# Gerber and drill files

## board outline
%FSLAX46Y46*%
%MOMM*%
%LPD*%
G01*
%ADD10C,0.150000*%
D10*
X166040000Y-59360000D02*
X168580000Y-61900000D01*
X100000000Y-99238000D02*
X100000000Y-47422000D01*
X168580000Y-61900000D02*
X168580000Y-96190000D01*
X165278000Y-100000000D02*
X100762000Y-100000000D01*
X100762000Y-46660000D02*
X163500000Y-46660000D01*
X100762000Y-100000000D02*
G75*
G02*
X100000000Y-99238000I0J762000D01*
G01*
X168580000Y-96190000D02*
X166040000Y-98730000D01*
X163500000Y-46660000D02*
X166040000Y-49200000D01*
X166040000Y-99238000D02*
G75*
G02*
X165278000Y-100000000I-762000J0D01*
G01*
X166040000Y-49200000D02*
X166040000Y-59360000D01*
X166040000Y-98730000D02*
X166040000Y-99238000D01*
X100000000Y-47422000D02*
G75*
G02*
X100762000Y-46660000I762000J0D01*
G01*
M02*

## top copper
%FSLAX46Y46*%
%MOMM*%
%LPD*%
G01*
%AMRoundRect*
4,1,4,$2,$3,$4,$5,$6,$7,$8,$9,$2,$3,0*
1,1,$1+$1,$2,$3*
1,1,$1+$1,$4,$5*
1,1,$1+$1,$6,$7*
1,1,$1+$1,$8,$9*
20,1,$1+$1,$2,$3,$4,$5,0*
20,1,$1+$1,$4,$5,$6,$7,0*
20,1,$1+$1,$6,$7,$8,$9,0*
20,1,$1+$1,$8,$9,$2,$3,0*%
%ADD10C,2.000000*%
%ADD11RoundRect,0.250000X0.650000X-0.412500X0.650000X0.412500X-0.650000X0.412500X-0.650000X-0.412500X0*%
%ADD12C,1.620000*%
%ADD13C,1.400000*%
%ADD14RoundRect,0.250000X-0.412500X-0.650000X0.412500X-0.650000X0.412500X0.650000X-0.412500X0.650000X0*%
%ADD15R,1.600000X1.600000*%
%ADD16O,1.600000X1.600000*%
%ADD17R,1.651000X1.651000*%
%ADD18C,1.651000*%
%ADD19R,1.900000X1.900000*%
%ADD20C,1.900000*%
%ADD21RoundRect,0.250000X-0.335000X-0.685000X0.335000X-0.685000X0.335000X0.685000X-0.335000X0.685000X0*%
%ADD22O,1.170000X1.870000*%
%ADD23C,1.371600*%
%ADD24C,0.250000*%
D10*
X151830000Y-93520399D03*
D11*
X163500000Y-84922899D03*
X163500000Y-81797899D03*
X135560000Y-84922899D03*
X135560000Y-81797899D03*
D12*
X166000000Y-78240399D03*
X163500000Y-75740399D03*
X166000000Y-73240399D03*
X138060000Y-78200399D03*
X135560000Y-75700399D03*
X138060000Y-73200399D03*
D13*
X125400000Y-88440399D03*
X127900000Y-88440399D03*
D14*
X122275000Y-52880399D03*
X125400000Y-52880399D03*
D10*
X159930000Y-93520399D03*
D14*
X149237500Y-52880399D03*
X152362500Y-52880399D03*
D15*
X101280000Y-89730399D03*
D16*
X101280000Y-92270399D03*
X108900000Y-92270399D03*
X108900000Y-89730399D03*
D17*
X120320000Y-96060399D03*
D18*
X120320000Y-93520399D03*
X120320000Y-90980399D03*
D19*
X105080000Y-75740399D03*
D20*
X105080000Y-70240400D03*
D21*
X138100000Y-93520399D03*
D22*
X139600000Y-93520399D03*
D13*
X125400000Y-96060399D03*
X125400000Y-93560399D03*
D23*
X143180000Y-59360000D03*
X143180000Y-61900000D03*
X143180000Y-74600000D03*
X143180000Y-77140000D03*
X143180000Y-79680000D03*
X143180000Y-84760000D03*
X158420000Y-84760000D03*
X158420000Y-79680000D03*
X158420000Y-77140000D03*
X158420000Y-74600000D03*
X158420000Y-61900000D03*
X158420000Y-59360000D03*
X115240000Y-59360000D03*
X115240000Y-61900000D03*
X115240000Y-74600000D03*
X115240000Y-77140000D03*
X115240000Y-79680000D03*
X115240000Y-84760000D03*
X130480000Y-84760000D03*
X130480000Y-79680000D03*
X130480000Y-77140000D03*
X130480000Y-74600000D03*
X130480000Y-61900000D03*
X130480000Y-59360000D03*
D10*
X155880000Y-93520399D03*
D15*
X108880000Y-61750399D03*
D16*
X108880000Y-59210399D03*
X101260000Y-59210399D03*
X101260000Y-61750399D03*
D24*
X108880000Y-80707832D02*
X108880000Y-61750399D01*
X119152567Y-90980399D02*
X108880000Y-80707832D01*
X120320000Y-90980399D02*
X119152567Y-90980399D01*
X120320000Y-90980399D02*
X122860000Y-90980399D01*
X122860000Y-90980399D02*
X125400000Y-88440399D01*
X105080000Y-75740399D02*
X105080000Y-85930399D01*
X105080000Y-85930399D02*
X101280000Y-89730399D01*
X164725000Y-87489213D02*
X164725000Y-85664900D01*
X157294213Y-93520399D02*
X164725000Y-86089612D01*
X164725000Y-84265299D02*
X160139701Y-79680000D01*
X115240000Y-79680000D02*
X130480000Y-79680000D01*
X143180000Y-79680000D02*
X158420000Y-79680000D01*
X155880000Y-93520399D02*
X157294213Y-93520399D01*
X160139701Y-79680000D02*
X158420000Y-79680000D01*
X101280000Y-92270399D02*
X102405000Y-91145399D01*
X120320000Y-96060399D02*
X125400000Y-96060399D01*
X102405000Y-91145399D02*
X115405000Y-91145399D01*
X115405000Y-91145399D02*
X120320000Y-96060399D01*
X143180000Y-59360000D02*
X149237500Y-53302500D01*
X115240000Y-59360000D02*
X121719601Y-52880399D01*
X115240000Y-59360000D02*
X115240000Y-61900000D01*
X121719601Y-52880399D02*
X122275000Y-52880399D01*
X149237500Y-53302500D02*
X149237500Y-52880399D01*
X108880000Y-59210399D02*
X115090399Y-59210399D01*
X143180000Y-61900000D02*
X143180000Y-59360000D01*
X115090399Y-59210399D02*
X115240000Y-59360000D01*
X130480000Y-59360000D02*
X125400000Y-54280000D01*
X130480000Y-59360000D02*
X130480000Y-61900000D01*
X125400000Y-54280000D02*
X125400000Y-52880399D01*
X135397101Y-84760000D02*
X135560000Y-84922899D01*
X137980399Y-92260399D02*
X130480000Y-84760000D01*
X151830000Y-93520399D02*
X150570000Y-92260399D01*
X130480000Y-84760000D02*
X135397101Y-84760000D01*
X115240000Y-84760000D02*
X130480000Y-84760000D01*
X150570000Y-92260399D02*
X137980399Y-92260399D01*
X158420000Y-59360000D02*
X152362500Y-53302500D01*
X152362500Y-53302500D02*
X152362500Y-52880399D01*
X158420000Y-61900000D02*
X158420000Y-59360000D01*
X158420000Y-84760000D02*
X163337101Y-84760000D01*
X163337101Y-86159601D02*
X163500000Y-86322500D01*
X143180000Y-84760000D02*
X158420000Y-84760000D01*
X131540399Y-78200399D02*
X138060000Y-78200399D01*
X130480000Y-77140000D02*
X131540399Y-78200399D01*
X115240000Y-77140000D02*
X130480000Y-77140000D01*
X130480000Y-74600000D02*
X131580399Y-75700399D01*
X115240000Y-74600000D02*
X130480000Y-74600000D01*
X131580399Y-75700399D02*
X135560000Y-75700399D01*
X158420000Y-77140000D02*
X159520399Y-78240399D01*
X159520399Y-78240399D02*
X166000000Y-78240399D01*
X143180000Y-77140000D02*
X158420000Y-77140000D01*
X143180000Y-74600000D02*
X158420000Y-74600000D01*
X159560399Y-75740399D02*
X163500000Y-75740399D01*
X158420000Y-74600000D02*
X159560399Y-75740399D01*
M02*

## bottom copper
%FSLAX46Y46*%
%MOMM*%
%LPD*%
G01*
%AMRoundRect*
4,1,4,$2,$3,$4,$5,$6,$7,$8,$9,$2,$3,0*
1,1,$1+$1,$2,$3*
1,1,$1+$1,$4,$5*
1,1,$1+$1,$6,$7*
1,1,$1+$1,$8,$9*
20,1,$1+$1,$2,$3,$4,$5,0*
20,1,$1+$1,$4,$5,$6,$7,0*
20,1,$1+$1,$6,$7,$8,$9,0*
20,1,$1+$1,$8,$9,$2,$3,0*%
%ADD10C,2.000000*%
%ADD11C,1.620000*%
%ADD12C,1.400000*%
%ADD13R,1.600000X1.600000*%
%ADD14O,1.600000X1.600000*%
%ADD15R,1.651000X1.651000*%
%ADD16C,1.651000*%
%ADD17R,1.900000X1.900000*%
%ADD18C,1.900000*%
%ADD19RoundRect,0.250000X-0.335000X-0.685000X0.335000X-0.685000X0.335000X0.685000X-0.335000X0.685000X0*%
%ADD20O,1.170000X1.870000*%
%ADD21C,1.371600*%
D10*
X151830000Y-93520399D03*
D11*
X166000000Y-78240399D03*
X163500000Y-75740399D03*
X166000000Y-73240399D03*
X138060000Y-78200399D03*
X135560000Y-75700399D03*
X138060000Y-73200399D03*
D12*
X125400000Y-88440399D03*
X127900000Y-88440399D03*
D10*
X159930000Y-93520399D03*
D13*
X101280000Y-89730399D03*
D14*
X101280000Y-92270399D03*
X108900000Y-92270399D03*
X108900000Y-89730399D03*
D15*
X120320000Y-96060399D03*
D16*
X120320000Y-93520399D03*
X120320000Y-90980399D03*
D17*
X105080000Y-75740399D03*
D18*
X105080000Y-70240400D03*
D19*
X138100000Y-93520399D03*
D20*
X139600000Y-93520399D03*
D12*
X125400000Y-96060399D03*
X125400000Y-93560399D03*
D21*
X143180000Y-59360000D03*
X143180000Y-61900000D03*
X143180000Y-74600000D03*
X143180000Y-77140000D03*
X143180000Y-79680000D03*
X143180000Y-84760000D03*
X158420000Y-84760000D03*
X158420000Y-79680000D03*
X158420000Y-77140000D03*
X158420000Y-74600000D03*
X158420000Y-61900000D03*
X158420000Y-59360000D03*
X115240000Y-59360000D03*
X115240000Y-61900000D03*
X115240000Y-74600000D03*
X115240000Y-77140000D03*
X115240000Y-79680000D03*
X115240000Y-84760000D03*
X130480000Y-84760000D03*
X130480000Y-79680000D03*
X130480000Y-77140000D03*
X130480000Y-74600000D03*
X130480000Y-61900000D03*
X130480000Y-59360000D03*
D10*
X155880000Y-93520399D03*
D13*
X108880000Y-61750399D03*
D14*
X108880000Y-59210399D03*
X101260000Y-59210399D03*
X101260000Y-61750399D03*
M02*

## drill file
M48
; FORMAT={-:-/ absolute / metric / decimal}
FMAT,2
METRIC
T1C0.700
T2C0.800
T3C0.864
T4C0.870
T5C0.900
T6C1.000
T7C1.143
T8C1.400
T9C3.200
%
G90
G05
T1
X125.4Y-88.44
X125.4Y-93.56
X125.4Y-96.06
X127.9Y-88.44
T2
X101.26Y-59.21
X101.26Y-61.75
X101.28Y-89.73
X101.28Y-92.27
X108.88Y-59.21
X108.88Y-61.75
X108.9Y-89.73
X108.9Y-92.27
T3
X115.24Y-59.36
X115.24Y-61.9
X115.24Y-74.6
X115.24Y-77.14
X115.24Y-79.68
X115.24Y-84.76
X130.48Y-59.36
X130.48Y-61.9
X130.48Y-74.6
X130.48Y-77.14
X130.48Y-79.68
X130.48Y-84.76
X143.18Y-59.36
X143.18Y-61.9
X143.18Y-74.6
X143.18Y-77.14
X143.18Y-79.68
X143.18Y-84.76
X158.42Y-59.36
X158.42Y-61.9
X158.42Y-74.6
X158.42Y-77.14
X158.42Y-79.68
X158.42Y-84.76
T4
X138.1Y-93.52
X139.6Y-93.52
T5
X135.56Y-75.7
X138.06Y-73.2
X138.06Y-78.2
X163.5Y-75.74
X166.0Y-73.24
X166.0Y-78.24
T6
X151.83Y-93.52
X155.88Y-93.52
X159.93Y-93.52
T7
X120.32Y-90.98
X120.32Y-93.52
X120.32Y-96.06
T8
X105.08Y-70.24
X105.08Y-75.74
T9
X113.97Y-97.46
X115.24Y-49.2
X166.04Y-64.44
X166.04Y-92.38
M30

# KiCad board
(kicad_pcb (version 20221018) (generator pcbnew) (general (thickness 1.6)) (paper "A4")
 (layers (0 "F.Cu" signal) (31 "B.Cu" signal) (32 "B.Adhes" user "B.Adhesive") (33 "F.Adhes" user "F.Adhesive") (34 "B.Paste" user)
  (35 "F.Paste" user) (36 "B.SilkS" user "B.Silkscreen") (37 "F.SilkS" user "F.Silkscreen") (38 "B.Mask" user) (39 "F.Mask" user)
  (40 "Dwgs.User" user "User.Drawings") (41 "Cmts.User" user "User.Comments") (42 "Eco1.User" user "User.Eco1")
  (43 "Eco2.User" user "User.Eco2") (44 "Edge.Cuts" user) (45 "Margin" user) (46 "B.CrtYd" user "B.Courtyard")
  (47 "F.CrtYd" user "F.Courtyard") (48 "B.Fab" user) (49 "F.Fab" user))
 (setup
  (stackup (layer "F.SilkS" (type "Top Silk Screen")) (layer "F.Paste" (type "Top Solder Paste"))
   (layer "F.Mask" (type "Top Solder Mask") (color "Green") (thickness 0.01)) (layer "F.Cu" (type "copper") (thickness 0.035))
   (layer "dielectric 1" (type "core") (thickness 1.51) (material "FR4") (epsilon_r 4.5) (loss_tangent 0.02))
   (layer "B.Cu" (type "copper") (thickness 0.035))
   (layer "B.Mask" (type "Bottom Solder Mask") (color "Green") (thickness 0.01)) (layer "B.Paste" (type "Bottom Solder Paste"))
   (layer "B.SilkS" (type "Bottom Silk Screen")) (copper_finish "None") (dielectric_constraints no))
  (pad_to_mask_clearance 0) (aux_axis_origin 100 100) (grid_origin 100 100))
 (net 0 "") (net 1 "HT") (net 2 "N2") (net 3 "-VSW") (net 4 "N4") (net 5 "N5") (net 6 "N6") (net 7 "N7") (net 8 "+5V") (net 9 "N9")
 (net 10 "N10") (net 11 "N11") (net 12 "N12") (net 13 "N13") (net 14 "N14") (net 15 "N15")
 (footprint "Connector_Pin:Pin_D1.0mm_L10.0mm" (layer "F.Cu") (at 151.83 93.520399 90)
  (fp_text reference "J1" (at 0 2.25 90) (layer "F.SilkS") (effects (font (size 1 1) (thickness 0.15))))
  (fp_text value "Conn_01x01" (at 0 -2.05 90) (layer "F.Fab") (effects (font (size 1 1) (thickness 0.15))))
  (pad "1" thru_hole circle (at 0 0 90) (size 2 2) (drill 1) (layers "*.Cu" "*.Mask") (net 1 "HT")))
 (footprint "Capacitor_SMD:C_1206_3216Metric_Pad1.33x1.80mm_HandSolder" (layer "F.Cu") (at 163.5 83.360399 90)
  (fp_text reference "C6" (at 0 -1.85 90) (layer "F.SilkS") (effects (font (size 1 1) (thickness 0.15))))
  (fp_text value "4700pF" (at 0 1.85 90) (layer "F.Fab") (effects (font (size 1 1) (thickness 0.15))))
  (pad "1" smd roundrect (at -1.5625 0 90) (size 1.325 1.8) (layers "F.Cu" "F.Paste" "F.Mask") (roundrect_rratio 0.188679) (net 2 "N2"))
  (pad "2" smd roundrect (at 1.5625 0 90) (size 1.325 1.8) (layers "F.Cu" "F.Paste" "F.Mask") (roundrect_rratio 0.188679) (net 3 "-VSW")))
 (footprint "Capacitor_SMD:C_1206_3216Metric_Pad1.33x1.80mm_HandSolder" (layer "F.Cu") (at 135.56 83.360399 90)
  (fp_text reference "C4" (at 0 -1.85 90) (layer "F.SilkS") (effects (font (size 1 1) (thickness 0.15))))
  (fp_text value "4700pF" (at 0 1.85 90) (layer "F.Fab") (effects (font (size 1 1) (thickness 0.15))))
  (pad "1" smd roundrect (at -1.5625 0 90) (size 1.325 1.8) (layers "F.Cu" "F.Paste" "F.Mask") (roundrect_rratio 0.188679) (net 1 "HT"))
  (pad "2" smd roundrect (at 1.5625 0 90) (size 1.325 1.8) (layers "F.Cu" "F.Paste" "F.Mask") (roundrect_rratio 0.188679) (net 3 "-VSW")))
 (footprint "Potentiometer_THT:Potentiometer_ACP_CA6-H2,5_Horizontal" (layer "F.Cu") (at 166 78.240399 180)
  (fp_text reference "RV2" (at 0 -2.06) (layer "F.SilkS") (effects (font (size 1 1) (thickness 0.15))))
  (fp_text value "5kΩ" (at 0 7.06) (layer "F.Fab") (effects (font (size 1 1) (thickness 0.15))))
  (pad "1" thru_hole circle (at 0 0 180) (size 1.62 1.62) (drill 0.9) (layers "*.Cu" "*.Mask") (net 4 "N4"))
  (pad "2" thru_hole circle (at 2.5 2.5 180) (size 1.62 1.62) (drill 0.9) (layers "*.Cu" "*.Mask") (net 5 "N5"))
  (pad "3" thru_hole circle (at 0 5 180) (size 1.62 1.62) (drill 0.9) (layers "*.Cu" "*.Mask") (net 3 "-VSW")))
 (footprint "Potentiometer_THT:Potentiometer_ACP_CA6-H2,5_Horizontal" (layer "F.Cu") (at 138.06 78.200399 180)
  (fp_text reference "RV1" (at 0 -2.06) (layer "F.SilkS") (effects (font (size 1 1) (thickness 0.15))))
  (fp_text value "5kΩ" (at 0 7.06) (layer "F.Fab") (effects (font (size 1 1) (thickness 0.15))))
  (pad "1" thru_hole circle (at 0 0 180) (size 1.62 1.62) (drill 0.9) (layers "*.Cu" "*.Mask") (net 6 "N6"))
  (pad "2" thru_hole circle (at 2.5 2.5 180) (size 1.62 1.62) (drill 0.9) (layers "*.Cu" "*.Mask") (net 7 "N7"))
  (pad "3" thru_hole circle (at 0 5 180) (size 1.62 1.62) (drill 0.9) (layers "*.Cu" "*.Mask") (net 3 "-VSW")))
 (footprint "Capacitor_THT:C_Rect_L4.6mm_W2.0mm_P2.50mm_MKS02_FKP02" (layer "F.Cu") (at 125.4 88.440399)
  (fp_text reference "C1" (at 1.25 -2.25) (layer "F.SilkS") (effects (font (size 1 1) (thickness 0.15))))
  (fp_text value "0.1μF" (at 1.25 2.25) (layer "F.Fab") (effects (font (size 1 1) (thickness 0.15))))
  (pad "1" thru_hole circle (at 0 0) (size 1.4 1.4) (drill 0.7) (layers "*.Cu" "*.Mask") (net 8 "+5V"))
  (pad "2" thru_hole circle (at 2.5 0) (size 1.4 1.4) (drill 0.7) (layers "*.Cu" "*.Mask") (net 3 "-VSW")))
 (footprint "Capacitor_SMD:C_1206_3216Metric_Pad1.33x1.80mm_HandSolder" (layer "F.Cu") (at 123.8375 52.880399)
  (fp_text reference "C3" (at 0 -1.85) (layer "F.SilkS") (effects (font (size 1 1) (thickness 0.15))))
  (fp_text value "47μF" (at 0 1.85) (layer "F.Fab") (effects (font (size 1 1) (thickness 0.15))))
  (pad "1" smd roundrect (at -1.5625 0) (size 1.325 1.8) (layers "F.Cu" "F.Paste" "F.Mask") (roundrect_rratio 0.188679) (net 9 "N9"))
  (pad "2" smd roundrect (at 1.5625 0) (size 1.325 1.8) (layers "F.Cu" "F.Paste" "F.Mask") (roundrect_rratio 0.188679) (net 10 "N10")))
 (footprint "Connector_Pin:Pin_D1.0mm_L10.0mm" (layer "F.Cu") (at 159.93 93.520399 90)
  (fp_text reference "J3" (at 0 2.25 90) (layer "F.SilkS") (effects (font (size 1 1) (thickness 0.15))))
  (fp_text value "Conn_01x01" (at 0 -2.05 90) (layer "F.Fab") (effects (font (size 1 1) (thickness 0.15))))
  (pad "1" thru_hole circle (at 0 0 90) (size 2 2) (drill 1) (layers "*.Cu" "*.Mask") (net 3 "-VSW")))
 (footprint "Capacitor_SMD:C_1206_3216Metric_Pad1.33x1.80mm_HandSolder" (layer "F.Cu") (at 150.8 52.880399)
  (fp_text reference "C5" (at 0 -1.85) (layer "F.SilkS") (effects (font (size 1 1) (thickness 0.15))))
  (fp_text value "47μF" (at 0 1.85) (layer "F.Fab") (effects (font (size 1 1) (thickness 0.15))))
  (pad "1" smd roundrect (at -1.5625 0) (size 1.325 1.8) (layers "F.Cu" "F.Paste" "F.Mask") (roundrect_rratio 0.188679) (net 9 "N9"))
  (pad "2" smd roundrect (at 1.5625 0) (size 1.325 1.8) (layers "F.Cu" "F.Paste" "F.Mask") (roundrect_rratio 0.188679) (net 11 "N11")))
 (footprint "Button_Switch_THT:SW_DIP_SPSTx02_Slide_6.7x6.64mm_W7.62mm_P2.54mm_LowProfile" (layer "F.Cu") (at 101.28 89.730399)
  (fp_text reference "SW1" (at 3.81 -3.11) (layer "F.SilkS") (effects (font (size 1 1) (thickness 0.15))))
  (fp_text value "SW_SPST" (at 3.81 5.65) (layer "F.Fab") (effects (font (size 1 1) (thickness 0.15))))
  (pad "1" thru_hole rect (at 0 0) (size 1.6 1.6) (drill 0.8) (layers "*.Cu" "*.Mask") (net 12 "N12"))
  (pad "2" thru_hole oval (at 0 2.54) (size 1.6 1.6) (drill 0.8) (layers "*.Cu" "*.Mask") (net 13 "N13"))
  (pad "3" thru_hole oval (at 7.62 2.54) (size 1.6 1.6) (drill 0.8) (layers "*.Cu" "*.Mask"))
  (pad "4" thru_hole oval (at 7.62 0) (size 1.6 1.6) (drill 0.8) (layers "*.Cu" "*.Mask")))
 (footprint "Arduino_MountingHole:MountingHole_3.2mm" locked (layer "F.Cu") (at 115.24 49.2)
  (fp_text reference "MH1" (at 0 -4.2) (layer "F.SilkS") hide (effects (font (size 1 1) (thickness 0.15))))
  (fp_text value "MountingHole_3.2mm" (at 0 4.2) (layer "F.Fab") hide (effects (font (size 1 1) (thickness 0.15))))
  (pad "" np_thru_hole circle locked (at 0 0) (size 3.2 3.2) (drill 3.2) (layers "*.Cu" "*.Mask")))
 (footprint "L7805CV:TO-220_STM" (layer "F.Cu") (at 120.32 96.060399 90)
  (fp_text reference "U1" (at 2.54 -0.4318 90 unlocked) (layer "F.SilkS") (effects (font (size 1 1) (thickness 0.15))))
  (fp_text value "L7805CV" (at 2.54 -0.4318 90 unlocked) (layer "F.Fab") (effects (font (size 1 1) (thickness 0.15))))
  (pad "1" thru_hole rect (at 0 0 90) (size 1.651 1.651) (drill 1.143) (layers "*.Cu" "*.Mask") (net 13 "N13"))
  (pad "2" thru_hole circle (at 2.54 0 90) (size 1.651 1.651) (drill 1.143) (layers "*.Cu" "*.Mask") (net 3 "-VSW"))
  (pad "3" thru_hole circle (at 5.08 0 90) (size 1.651 1.651) (drill 1.143) (layers "*.Cu" "*.Mask") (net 8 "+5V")))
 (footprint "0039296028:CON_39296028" (layer "F.Cu") (at 105.08 75.740399 180)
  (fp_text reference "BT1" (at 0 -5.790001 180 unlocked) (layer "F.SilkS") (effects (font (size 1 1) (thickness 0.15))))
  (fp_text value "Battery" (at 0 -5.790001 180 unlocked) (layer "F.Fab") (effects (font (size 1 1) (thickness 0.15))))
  (pad "1" thru_hole rect (at 0 0 180) (size 1.9 1.9) (drill 1.4) (layers "*.Cu" "*.Mask") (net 12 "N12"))
  (pad "2" thru_hole circle (at 0 5.499999 180) (size 1.9 1.9) (drill 1.4) (layers "*.Cu" "*.Mask") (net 3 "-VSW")))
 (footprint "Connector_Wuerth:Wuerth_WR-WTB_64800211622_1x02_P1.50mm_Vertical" (layer "F.Cu") (at 138.1 93.520399)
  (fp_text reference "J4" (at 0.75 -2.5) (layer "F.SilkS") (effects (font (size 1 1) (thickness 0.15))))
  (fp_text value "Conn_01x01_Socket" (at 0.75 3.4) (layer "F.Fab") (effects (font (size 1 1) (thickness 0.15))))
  (pad "1" thru_hole roundrect (at 0 0) (size 1.17 1.87) (drill 0.87) (layers "*.Cu" "*.Mask") (roundrect_rratio 0.213675) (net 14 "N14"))
  (pad "2" thru_hole oval (at 1.5 0) (size 1.17 1.87) (drill 0.87) (layers "*.Cu" "*.Mask") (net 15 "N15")))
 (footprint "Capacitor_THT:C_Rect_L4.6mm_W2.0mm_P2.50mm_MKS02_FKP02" (layer "F.Cu") (at 125.4 96.060399 90)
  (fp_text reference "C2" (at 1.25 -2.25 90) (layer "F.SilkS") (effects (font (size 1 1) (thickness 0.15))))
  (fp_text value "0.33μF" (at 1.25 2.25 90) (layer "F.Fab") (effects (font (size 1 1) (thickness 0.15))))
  (pad "1" thru_hole circle (at 0 0 90) (size 1.4 1.4) (drill 0.7) (layers "*.Cu" "*.Mask") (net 13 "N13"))
  (pad "2" thru_hole circle (at 2.5 0 90) (size 1.4 1.4) (drill 0.7) (layers "*.Cu" "*.Mask") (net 3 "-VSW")))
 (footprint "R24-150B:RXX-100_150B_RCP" (layer "F.Cu") (at 143.18 59.36)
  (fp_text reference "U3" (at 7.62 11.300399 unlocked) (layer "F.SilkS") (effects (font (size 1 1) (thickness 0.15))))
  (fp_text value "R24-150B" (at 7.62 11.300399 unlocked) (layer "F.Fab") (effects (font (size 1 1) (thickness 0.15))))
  (pad "2" thru_hole circle (at 0 0) (size 1.3716 1.3716) (drill 0.8636) (layers "*.Cu" "*.Mask") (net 9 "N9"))
  (pad "3" thru_hole circle (at 0 2.54) (size 1.3716 1.3716) (drill 0.8636) (layers "*.Cu" "*.Mask") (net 9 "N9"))
  (pad "8" thru_hole circle (at 0 15.24) (size 1.3716 1.3716) (drill 0.8636) (layers "*.Cu" "*.Mask") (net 5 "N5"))
  (pad "9" thru_hole circle (at 0 17.78) (size 1.3716 1.3716) (drill 0.8636) (layers "*.Cu" "*.Mask") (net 4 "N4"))
  (pad "10" thru_hole circle (at 0 20.32) (size 1.3716 1.3716) (drill 0.8636) (layers "*.Cu" "*.Mask") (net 3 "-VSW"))
  (pad "12" thru_hole circle (at 0 25.4) (size 1.3716 1.3716) (drill 0.8636) (layers "*.Cu" "*.Mask") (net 2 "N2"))
  (pad "13" thru_hole circle (at 15.24 25.4) (size 1.3716 1.3716) (drill 0.8636) (layers "*.Cu" "*.Mask") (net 2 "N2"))
  (pad "15" thru_hole circle (at 15.24 20.32) (size 1.3716 1.3716) (drill 0.8636) (layers "*.Cu" "*.Mask") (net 3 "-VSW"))
  (pad "16" thru_hole circle (at 15.24 17.78) (size 1.3716 1.3716) (drill 0.8636) (layers "*.Cu" "*.Mask") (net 4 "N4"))
  (pad "17" thru_hole circle (at 15.24 15.24) (size 1.3716 1.3716) (drill 0.8636) (layers "*.Cu" "*.Mask") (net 5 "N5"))
  (pad "22" thru_hole circle (at 15.24 2.54) (size 1.3716 1.3716) (drill 0.8636) (layers "*.Cu" "*.Mask") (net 11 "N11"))
  (pad "23" thru_hole circle (at 15.24 0) (size 1.3716 1.3716) (drill 0.8636) (layers "*.Cu" "*.Mask") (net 11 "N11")))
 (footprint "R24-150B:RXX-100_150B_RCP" (layer "F.Cu") (at 115.24 59.36)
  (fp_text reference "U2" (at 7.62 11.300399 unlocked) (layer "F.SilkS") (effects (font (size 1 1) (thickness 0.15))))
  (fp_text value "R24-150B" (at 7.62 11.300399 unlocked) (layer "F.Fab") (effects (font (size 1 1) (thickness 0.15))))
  (pad "2" thru_hole circle (at 0 0) (size 1.3716 1.3716) (drill 0.8636) (layers "*.Cu" "*.Mask") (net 9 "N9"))
  (pad "3" thru_hole circle (at 0 2.54) (size 1.3716 1.3716) (drill 0.8636) (layers "*.Cu" "*.Mask") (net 9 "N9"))
  (pad "8" thru_hole circle (at 0 15.24) (size 1.3716 1.3716) (drill 0.8636) (layers "*.Cu" "*.Mask") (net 7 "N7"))
  (pad "9" thru_hole circle (at 0 17.78) (size 1.3716 1.3716) (drill 0.8636) (layers "*.Cu" "*.Mask") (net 6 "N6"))
  (pad "10" thru_hole circle (at 0 20.32) (size 1.3716 1.3716) (drill 0.8636) (layers "*.Cu" "*.Mask") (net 3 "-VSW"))
  (pad "12" thru_hole circle (at 0 25.4) (size 1.3716 1.3716) (drill 0.8636) (layers "*.Cu" "*.Mask") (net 1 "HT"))
  (pad "13" thru_hole circle (at 15.24 25.4) (size 1.3716 1.3716) (drill 0.8636) (layers "*.Cu" "*.Mask") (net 1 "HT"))
  (pad "15" thru_hole circle (at 15.24 20.32) (size 1.3716 1.3716) (drill 0.8636) (layers "*.Cu" "*.Mask") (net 3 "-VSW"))
  (pad "16" thru_hole circle (at 15.24 17.78) (size 1.3716 1.3716) (drill 0.8636) (layers "*.Cu" "*.Mask") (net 6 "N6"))
  (pad "17" thru_hole circle (at 15.24 15.24) (size 1.3716 1.3716) (drill 0.8636) (layers "*.Cu" "*.Mask") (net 7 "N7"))
  (pad "22" thru_hole circle (at 15.24 2.54) (size 1.3716 1.3716) (drill 0.8636) (layers "*.Cu" "*.Mask") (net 10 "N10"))
  (pad "23" thru_hole circle (at 15.24 0) (size 1.3716 1.3716) (drill 0.8636) (layers "*.Cu" "*.Mask") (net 10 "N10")))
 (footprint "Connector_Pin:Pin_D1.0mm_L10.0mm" (layer "F.Cu") (at 155.88 93.520399 90)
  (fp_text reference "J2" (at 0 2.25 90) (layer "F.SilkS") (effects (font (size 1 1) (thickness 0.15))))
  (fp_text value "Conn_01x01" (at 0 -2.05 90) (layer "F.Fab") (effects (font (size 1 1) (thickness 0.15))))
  (pad "1" thru_hole circle (at 0 0 90) (size 2 2) (drill 1) (layers "*.Cu" "*.Mask") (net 3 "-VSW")))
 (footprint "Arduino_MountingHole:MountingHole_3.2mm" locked (layer "F.Cu") (at 113.97 97.46)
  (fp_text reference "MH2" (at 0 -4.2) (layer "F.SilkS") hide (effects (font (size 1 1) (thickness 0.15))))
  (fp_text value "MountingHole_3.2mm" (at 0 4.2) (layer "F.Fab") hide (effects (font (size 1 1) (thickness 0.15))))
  (pad "" np_thru_hole circle locked (at 0 0) (size 3.2 3.2) (drill 3.2) (layers "*.Cu" "*.Mask")))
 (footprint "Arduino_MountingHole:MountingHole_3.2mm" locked (layer "F.Cu") (at 166.04 64.44)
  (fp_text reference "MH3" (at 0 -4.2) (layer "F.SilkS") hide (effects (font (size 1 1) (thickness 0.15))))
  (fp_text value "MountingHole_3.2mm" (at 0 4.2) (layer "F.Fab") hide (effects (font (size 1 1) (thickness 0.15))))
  (pad "" np_thru_hole circle locked (at 0 0) (size 3.2 3.2) (drill 3.2) (layers "*.Cu" "*.Mask")))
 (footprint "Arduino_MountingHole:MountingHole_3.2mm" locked (layer "F.Cu") (at 166.04 92.38)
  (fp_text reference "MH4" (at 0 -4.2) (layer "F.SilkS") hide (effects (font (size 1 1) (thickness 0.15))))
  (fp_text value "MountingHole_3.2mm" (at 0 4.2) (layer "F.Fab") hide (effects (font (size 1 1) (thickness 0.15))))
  (pad "" np_thru_hole circle locked (at 0 0) (size 3.2 3.2) (drill 3.2) (layers "*.Cu" "*.Mask")))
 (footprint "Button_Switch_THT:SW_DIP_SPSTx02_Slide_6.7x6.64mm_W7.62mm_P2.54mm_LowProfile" (layer "F.Cu") (at 108.88 61.750399 180)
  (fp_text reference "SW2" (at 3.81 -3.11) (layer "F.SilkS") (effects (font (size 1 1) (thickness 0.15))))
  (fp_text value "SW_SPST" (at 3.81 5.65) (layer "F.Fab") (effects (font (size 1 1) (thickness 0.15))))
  (pad "1" thru_hole rect (at 0 0 180) (size 1.6 1.6) (drill 0.8) (layers "*.Cu" "*.Mask") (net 8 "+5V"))
  (pad "2" thru_hole oval (at 0 2.54 180) (size 1.6 1.6) (drill 0.8) (layers "*.Cu" "*.Mask") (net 9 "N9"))
  (pad "3" thru_hole oval (at 7.62 2.54 180) (size 1.6 1.6) (drill 0.8) (layers "*.Cu" "*.Mask"))
  (pad "4" thru_hole oval (at 7.62 0 180) (size 1.6 1.6) (drill 0.8) (layers "*.Cu" "*.Mask")))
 (gr_line (start 166.04 59.36) (end 168.58 61.9) (stroke (width 0.15) (type solid)) (layer "Edge.Cuts"))
 (gr_line (start 100 99.238) (end 100 47.422) (stroke (width 0.15) (type solid)) (layer "Edge.Cuts"))
 (gr_line (start 168.58 61.9) (end 168.58 96.19) (stroke (width 0.15) (type solid)) (layer "Edge.Cuts"))
 (gr_line (start 165.278 100) (end 100.762 100) (stroke (width 0.15) (type solid)) (layer "Edge.Cuts"))
 (gr_line (start 100.762 46.66) (end 163.5 46.66) (stroke (width 0.15) (type solid)) (layer "Edge.Cuts"))
 (gr_arc (start 100.762 100) (mid 100.223185 99.776815) (end 100 99.238) (stroke (width 0.15) (type solid)) (layer "Edge.Cuts"))
 (gr_line (start 168.58 96.19) (end 166.04 98.73) (stroke (width 0.15) (type solid)) (layer "Edge.Cuts"))
 (gr_line (start 163.5 46.66) (end 166.04 49.2) (stroke (width 0.15) (type solid)) (layer "Edge.Cuts"))
 (gr_arc (start 166.04 99.238) (mid 165.816815 99.776815) (end 165.278 100) (stroke (width 0.15) (type solid)) (layer "Edge.Cuts"))
 (gr_line (start 166.04 49.2) (end 166.04 59.36) (stroke (width 0.15) (type solid)) (layer "Edge.Cuts"))
 (gr_line (start 166.04 98.73) (end 166.04 99.238) (stroke (width 0.15) (type solid)) (layer "Edge.Cuts"))
 (gr_arc (start 100 47.422) (mid 100.223185 46.883185) (end 100.762 46.66) (stroke (width 0.15) (type solid)) (layer "Edge.Cuts"))
 (segment (start 108.88 80.707832) (end 108.88 61.750399) (width 0.25) (layer "F.Cu") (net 8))
 (segment (start 119.152567 90.980399) (end 108.88 80.707832) (width 0.25) (layer "F.Cu") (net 8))
 (segment (start 120.32 90.980399) (end 119.152567 90.980399) (width 0.25) (layer "F.Cu") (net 8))
 (segment (start 120.32 90.980399) (end 122.86 90.980399) (width 0.25) (layer "F.Cu") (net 8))
 (segment (start 122.86 90.980399) (end 125.4 88.440399) (width 0.25) (layer "F.Cu") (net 8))
 (segment (start 105.08 75.740399) (end 105.08 85.930399) (width 0.25) (layer "F.Cu") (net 12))
 (segment (start 105.08 85.930399) (end 101.28 89.730399) (width 0.25) (layer "F.Cu") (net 12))
 (segment (start 164.725 87.489213) (end 164.725 85.6649) (width 0.25) (layer "F.Cu") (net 3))
 (segment (start 157.294213 93.520399) (end 164.725 86.089612) (width 0.25) (layer "F.Cu") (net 3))
 (segment (start 164.725 84.265299) (end 160.139701 79.68) (width 0.25) (layer "F.Cu") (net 3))
 (segment (start 115.24 79.68) (end 130.48 79.68) (width 0.25) (layer "F.Cu") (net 3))
 (segment (start 143.18 79.68) (end 158.42 79.68) (width 0.25) (layer "F.Cu") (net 3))
 (segment (start 155.88 93.520399) (end 157.294213 93.520399) (width 0.25) (layer "F.Cu") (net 3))
 (segment (start 160.139701 79.68) (end 158.42 79.68) (width 0.25) (layer "F.Cu") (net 3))
 (segment (start 101.28 92.270399) (end 102.405 91.145399) (width 0.25) (layer "F.Cu") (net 13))
 (segment (start 120.32 96.060399) (end 125.4 96.060399) (width 0.25) (layer "F.Cu") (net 13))
 (segment (start 102.405 91.145399) (end 115.405 91.145399) (width 0.25) (layer "F.Cu") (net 13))
 (segment (start 115.405 91.145399) (end 120.32 96.060399) (width 0.25) (layer "F.Cu") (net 13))
 (segment (start 143.18 59.36) (end 149.2375 53.3025) (width 0.25) (layer "F.Cu") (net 9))
 (segment (start 115.24 59.36) (end 121.719601 52.880399) (width 0.25) (layer "F.Cu") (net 9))
 (segment (start 115.24 59.36) (end 115.24 61.9) (width 0.25) (layer "F.Cu") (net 9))
 (segment (start 121.719601 52.880399) (end 122.275 52.880399) (width 0.25) (layer "F.Cu") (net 9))
 (segment (start 149.2375 53.3025) (end 149.2375 52.880399) (width 0.25) (layer "F.Cu") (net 9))
 (segment (start 108.88 59.210399) (end 115.090399 59.210399) (width 0.25) (layer "F.Cu") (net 9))
 (segment (start 143.18 61.9) (end 143.18 59.36) (width 0.25) (layer "F.Cu") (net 9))
 (segment (start 115.090399 59.210399) (end 115.24 59.36) (width 0.25) (layer "F.Cu") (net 9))
 (segment (start 130.48 59.36) (end 125.4 54.28) (width 0.25) (layer "F.Cu") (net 10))
 (segment (start 130.48 59.36) (end 130.48 61.9) (width 0.25) (layer "F.Cu") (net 10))
 (segment (start 125.4 54.28) (end 125.4 52.880399) (width 0.25) (layer "F.Cu") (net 10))
 (segment (start 135.397101 84.76) (end 135.56 84.922899) (width 0.25) (layer "F.Cu") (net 1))
 (segment (start 137.980399 92.260399) (end 130.48 84.76) (width 0.25) (layer "F.Cu") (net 1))
 (segment (start 151.83 93.520399) (end 150.57 92.260399) (width 0.25) (layer "F.Cu") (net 1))
 (segment (start 130.48 84.76) (end 135.397101 84.76) (width 0.25) (layer "F.Cu") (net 1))
 (segment (start 115.24 84.76) (end 130.48 84.76) (width 0.25) (layer "F.Cu") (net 1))
 (segment (start 150.57 92.260399) (end 137.980399 92.260399) (width 0.25) (layer "F.Cu") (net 1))
 (segment (start 158.42 59.36) (end 152.3625 53.3025) (width 0.25) (layer "F.Cu") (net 11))
 (segment (start 152.3625 53.3025) (end 152.3625 52.880399) (width 0.25) (layer "F.Cu") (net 11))
 (segment (start 158.42 61.9) (end 158.42 59.36) (width 0.25) (layer "F.Cu") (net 11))
 (segment (start 158.42 84.76) (end 163.337101 84.76) (width 0.25) (layer "F.Cu") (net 2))
 (segment (start 163.337101 86.159601) (end 163.5 86.3225) (width 0.25) (layer "F.Cu") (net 2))
 (segment (start 143.18 84.76) (end 158.42 84.76) (width 0.25) (layer "F.Cu") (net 2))
 (segment (start 131.540399 78.200399) (end 138.06 78.200399) (width 0.25) (layer "F.Cu") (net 6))
 (segment (start 130.48 77.14) (end 131.540399 78.200399) (width 0.25) (layer "F.Cu") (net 6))
 (segment (start 115.24 77.14) (end 130.48 77.14) (width 0.25) (layer "F.Cu") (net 6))
 (segment (start 130.48 74.6) (end 131.580399 75.700399) (width 0.25) (layer "F.Cu") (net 7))
 (segment (start 115.24 74.6) (end 130.48 74.6) (width 0.25) (layer "F.Cu") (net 7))
 (segment (start 131.580399 75.700399) (end 135.56 75.700399) (width 0.25) (layer "F.Cu") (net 7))
 (segment (start 158.42 77.14) (end 159.520399 78.240399) (width 0.25) (layer "F.Cu") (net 4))
 (segment (start 159.520399 78.240399) (end 166 78.240399) (width 0.25) (layer "F.Cu") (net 4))
 (segment (start 143.18 77.14) (end 158.42 77.14) (width 0.25) (layer "F.Cu") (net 4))
 (segment (start 143.18 74.6) (end 158.42 74.6) (width 0.25) (layer "F.Cu") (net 5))
 (segment (start 159.560399 75.740399) (end 163.5 75.740399) (width 0.25) (layer "F.Cu") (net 5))
 (segment (start 158.42 74.6) (end 159.560399 75.740399) (width 0.25) (layer "F.Cu") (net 5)))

